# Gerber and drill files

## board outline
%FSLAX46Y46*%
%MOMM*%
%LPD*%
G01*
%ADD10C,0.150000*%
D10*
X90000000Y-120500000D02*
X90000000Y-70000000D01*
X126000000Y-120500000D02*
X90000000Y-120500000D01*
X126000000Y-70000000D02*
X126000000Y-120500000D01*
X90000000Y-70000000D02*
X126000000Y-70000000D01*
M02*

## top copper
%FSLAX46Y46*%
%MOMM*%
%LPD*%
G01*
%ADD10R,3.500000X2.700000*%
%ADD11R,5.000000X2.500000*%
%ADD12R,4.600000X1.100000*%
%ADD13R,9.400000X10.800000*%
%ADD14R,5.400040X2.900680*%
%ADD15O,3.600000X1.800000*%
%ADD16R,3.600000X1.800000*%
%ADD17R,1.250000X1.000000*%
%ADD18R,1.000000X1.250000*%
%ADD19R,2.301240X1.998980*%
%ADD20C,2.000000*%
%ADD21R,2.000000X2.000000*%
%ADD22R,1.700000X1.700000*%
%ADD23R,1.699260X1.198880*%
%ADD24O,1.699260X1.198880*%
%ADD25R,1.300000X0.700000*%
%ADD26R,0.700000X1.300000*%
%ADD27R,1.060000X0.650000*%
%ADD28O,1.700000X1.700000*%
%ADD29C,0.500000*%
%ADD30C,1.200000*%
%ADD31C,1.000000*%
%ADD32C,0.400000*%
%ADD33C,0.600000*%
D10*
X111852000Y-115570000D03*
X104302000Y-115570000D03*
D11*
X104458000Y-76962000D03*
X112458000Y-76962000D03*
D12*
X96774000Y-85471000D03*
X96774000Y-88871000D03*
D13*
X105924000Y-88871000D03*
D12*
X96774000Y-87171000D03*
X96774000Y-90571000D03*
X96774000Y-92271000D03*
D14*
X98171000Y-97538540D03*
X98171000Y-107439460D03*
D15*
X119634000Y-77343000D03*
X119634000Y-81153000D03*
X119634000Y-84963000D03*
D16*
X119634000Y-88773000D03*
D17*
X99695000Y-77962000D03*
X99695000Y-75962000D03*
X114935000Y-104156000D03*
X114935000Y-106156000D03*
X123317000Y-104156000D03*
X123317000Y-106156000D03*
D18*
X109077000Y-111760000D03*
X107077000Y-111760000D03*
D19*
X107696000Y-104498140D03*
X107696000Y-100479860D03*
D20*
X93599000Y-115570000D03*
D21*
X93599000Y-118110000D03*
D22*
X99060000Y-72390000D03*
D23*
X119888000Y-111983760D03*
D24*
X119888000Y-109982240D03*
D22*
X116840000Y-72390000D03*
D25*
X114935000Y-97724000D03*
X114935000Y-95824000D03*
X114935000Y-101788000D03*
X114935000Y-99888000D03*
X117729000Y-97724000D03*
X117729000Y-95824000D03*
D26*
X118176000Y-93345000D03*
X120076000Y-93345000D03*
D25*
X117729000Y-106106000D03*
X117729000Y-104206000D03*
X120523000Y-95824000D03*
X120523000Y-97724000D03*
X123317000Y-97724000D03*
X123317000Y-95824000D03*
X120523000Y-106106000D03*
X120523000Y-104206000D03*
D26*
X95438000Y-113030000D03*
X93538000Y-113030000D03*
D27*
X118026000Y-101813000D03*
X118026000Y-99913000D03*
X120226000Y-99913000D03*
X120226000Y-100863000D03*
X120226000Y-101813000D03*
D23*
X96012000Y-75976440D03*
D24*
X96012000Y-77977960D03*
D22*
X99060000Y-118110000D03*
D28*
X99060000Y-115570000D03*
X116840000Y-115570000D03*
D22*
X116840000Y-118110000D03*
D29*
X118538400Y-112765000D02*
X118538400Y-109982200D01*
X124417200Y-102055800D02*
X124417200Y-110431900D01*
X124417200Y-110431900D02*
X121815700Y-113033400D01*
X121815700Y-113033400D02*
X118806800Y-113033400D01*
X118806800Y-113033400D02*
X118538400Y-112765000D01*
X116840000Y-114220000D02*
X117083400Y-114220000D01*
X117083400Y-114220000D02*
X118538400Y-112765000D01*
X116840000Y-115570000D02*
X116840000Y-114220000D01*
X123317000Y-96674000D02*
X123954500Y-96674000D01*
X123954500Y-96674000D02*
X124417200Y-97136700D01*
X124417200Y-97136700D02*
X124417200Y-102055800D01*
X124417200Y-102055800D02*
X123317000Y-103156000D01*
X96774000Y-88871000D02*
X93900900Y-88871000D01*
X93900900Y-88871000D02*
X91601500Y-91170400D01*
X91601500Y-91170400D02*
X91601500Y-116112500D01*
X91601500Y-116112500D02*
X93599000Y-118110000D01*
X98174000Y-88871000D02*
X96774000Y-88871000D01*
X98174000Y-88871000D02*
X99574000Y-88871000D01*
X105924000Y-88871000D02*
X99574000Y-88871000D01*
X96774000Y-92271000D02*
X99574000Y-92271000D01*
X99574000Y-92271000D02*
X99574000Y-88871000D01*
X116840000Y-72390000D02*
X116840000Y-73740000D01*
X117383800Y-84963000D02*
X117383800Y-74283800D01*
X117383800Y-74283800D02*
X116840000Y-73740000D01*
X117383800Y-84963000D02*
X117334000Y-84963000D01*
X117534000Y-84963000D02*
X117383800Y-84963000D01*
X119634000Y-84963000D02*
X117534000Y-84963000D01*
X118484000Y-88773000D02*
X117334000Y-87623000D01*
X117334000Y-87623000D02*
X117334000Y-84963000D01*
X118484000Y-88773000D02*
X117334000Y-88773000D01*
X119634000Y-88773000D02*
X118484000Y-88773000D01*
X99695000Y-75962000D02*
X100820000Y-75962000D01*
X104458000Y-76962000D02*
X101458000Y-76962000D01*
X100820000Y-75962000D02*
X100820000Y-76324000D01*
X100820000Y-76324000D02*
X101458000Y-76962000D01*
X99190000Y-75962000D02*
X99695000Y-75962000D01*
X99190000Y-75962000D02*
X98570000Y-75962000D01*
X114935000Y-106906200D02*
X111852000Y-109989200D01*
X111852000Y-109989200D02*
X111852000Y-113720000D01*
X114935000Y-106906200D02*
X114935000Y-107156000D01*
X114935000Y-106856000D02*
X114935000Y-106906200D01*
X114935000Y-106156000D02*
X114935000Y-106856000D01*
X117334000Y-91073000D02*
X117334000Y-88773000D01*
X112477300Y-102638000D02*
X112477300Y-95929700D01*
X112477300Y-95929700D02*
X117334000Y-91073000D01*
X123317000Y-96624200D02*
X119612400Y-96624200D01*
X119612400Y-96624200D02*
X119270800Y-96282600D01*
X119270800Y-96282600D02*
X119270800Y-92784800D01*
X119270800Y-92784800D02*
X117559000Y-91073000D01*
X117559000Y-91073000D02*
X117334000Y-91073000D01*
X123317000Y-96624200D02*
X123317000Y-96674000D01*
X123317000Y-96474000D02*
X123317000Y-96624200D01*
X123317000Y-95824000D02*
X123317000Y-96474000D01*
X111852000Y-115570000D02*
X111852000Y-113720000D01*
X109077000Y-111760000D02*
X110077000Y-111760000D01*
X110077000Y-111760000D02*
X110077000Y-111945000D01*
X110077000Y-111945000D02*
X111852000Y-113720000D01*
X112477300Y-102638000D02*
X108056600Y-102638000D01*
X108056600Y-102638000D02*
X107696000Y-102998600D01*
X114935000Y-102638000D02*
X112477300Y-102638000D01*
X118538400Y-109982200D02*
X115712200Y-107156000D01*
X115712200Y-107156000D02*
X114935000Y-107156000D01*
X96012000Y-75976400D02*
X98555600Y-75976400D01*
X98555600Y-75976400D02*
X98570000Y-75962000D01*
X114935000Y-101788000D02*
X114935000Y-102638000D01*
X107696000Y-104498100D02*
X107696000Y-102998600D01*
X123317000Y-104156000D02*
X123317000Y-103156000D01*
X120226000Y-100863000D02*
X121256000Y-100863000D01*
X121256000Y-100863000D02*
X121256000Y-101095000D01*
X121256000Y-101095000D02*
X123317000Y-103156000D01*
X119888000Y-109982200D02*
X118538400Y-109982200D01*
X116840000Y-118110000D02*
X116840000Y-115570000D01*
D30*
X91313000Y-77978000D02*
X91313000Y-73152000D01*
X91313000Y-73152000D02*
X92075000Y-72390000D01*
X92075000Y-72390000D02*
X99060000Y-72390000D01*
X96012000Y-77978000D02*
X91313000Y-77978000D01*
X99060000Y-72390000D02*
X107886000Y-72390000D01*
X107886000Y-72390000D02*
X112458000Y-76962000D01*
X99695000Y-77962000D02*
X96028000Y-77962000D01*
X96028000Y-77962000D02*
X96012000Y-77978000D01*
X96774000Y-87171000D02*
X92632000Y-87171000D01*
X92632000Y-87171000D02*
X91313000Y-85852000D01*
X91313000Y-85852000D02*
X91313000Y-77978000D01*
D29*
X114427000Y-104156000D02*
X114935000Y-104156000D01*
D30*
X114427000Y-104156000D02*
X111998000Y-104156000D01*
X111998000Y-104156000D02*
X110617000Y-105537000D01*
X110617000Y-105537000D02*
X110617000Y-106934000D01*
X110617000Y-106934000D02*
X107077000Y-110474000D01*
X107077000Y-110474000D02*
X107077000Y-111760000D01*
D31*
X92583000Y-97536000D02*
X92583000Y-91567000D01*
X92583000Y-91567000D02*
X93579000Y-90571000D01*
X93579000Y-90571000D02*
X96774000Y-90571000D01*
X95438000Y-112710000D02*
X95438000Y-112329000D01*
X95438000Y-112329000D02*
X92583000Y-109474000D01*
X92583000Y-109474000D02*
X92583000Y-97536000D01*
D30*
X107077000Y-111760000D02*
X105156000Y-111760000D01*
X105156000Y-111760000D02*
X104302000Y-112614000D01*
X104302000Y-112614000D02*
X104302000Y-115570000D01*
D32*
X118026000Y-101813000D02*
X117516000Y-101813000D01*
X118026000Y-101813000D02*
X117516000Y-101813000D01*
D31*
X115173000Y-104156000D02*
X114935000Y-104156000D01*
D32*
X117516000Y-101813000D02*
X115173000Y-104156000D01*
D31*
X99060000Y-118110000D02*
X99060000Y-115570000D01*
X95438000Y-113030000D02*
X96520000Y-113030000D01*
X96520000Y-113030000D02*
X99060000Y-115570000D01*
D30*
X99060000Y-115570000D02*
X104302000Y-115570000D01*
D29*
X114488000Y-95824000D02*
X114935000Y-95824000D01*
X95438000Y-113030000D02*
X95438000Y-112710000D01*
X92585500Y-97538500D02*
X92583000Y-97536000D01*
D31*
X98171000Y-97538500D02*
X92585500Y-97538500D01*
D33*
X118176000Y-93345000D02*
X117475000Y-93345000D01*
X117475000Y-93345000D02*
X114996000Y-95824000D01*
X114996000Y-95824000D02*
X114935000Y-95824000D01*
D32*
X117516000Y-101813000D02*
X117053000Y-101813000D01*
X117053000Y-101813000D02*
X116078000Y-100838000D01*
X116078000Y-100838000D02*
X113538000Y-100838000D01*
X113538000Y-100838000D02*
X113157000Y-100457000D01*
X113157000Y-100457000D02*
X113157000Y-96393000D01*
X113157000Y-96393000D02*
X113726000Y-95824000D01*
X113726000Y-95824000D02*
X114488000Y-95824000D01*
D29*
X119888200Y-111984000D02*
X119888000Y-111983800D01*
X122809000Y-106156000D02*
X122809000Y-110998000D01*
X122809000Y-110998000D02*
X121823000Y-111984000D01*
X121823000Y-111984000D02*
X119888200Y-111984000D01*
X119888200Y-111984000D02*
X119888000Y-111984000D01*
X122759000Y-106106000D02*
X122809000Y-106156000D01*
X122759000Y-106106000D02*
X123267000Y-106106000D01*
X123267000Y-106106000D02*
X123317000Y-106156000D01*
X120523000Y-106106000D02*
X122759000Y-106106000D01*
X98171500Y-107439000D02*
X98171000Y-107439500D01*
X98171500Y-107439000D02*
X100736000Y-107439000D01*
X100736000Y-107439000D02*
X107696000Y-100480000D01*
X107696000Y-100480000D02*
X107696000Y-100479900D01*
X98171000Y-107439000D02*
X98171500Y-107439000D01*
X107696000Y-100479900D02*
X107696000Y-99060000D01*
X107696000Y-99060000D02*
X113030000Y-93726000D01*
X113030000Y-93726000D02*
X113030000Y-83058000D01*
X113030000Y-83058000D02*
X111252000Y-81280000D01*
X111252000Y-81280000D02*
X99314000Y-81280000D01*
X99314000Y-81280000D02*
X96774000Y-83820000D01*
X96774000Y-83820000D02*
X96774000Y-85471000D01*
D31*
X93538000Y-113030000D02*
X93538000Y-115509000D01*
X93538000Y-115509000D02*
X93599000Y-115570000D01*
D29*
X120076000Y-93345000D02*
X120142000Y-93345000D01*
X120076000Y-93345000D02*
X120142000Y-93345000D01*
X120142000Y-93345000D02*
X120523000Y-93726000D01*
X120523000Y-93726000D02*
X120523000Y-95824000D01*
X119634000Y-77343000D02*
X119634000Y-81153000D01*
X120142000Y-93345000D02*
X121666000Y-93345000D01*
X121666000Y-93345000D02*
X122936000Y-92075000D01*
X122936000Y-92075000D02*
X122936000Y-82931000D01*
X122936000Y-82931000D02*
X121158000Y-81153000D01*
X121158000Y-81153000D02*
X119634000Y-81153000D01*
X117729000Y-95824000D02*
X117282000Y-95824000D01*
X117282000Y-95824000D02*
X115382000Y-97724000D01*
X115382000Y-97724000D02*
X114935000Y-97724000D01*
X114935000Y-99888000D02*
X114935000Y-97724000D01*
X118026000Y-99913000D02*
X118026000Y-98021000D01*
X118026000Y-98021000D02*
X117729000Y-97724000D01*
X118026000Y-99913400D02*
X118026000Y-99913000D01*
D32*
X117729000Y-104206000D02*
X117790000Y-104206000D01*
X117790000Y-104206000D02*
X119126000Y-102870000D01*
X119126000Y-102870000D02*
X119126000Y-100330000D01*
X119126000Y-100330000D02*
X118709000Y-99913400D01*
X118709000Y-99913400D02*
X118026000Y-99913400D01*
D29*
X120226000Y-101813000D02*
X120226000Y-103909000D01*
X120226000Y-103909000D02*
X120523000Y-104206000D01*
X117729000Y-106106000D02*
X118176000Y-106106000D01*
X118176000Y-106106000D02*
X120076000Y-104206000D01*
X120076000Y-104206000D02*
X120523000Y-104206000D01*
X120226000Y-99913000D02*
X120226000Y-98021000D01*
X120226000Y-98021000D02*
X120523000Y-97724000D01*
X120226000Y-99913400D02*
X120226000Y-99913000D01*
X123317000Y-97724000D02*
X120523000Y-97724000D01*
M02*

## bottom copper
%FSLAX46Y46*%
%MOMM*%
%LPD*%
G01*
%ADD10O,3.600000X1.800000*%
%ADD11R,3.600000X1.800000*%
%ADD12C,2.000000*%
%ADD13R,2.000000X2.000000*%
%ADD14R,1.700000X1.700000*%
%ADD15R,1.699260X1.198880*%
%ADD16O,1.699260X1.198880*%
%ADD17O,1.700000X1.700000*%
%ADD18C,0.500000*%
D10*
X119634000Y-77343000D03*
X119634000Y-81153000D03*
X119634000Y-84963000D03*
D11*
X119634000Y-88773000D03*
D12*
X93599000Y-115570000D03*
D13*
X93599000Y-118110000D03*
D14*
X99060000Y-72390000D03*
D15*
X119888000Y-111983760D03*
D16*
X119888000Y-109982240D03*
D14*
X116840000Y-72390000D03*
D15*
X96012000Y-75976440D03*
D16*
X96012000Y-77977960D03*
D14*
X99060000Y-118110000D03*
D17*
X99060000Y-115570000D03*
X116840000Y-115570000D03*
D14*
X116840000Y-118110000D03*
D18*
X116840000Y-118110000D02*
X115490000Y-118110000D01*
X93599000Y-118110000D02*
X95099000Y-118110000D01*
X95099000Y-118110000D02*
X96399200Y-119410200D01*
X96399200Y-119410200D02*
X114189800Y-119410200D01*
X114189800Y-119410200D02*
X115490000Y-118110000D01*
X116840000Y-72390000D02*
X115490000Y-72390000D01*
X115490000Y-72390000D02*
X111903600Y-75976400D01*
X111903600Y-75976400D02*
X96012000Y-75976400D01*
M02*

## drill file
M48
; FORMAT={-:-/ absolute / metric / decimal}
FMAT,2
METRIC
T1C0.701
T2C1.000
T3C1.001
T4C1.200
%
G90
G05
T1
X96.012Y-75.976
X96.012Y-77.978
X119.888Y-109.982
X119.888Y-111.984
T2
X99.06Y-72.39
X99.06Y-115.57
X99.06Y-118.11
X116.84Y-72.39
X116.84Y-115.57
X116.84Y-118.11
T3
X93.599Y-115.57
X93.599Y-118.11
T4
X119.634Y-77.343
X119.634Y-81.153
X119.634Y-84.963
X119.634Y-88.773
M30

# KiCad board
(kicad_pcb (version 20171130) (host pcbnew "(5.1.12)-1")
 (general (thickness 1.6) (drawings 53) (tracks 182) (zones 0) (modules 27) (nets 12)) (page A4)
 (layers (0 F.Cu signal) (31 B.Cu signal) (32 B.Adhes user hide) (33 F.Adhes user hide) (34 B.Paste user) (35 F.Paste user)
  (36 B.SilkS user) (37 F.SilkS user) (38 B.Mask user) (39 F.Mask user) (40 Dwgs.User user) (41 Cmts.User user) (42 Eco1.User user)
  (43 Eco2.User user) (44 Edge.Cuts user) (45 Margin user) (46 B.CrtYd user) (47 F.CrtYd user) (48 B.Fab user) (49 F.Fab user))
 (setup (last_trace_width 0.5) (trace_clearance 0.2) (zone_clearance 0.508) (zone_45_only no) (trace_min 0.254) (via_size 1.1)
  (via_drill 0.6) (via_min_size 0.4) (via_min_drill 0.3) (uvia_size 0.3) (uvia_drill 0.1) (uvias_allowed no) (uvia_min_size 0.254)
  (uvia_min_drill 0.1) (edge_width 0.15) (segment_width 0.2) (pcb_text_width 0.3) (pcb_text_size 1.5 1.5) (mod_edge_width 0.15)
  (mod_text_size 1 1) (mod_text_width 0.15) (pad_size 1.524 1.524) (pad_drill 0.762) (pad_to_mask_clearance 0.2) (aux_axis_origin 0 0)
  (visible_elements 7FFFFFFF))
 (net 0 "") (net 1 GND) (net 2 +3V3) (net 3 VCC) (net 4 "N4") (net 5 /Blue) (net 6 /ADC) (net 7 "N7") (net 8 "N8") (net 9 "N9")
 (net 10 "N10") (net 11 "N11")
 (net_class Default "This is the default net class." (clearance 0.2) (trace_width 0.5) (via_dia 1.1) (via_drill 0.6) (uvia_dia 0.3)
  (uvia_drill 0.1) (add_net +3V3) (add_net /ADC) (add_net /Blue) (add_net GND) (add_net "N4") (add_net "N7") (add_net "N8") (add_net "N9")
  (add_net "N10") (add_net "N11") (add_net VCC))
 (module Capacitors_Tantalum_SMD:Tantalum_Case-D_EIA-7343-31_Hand (layer F.Cu) (at 108.077 115.57)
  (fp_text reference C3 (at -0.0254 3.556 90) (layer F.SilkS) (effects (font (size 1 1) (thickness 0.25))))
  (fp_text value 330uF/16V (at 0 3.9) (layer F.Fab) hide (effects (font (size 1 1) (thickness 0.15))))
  (pad 2 smd rect (at 3.775 0) (size 3.5 2.7) (layers F.Cu F.Paste F.Mask) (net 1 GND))
  (pad 1 smd rect (at -3.775 0) (size 3.5 2.7) (layers F.Cu F.Paste F.Mask) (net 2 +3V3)))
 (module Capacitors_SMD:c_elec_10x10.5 (layer F.Cu) (at 108.458 76.962 180)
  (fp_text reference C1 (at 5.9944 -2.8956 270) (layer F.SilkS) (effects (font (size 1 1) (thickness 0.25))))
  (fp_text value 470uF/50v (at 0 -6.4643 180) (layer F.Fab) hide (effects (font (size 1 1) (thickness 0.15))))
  (pad 2 smd rect (at 4 0) (size 5 2.5) (layers F.Cu F.Paste F.Mask) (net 1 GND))
  (pad 1 smd rect (at -4 0) (size 5 2.5) (layers F.Cu F.Paste F.Mask) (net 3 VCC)))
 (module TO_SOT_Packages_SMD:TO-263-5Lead (layer F.Cu) (at 96.774 88.871)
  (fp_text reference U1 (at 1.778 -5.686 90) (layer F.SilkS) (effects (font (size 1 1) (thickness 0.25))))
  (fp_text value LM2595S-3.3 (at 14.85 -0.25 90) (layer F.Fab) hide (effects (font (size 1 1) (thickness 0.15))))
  (pad 1 smd rect (at 0 -3.4) (size 4.6 1.1) (layers F.Cu F.Paste F.Mask) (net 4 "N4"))
  (pad 3 smd rect (at 0 0) (size 4.6 1.1) (layers F.Cu F.Paste F.Mask) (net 1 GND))
  (pad 3 smd rect (at 9.15 0) (size 9.4 10.8) (layers F.Cu F.Paste F.Mask) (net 1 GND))
  (pad 2 smd rect (at 0 -1.7) (size 4.6 1.1) (layers F.Cu F.Paste F.Mask) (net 3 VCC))
  (pad 4 smd rect (at 0 1.7) (size 4.6 1.1) (layers F.Cu F.Paste F.Mask) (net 2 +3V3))
  (pad 5 smd rect (at 0 3.4) (size 4.6 1.1) (layers F.Cu F.Paste F.Mask) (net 1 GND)))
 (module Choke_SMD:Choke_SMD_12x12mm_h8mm (layer F.Cu) (at 98.171 102.489 90)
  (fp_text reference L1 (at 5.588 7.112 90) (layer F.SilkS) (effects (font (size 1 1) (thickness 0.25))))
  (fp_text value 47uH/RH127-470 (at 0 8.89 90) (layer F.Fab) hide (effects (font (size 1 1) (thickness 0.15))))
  (pad 2 smd rect (at 4.95046 0 90) (size 2.90068 5.40004) (layers F.Cu F.Paste F.Mask) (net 2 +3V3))
  (pad 1 smd rect (at -4.95046 0 90) (size 2.90068 5.40004) (layers F.Cu F.Paste F.Mask) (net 4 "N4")))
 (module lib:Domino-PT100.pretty (layer F.Cu) (at 119.634 88.773 90)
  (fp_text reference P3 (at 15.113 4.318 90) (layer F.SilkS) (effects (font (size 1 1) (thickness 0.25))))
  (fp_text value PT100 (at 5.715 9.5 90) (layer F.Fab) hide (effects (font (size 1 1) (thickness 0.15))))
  (pad 4 thru_hole oval (at 11.43 0 90) (size 1.8 3.6) (drill 1.2) (layers *.Cu *.Mask) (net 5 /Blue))
  (pad 3 thru_hole oval (at 7.62 0 90) (size 1.8 3.6) (drill 1.2) (layers *.Cu *.Mask) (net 5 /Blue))
  (pad 2 thru_hole oval (at 3.81 0 90) (size 1.8 3.6) (drill 1.2) (layers *.Cu *.Mask) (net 1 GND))
  (pad 1 thru_hole rect (at 0 0 90) (size 1.8 3.6) (drill 1.2) (layers *.Cu *.Mask) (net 1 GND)))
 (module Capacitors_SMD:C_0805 (layer F.Cu) (at 99.695 76.962 90)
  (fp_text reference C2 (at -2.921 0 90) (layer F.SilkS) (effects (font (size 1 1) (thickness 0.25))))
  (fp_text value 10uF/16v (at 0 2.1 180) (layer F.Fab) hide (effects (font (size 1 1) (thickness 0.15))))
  (pad 1 smd rect (at -1 0 90) (size 1 1.25) (layers F.Cu F.Paste F.Mask) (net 3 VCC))
  (pad 2 smd rect (at 1 0 90) (size 1 1.25) (layers F.Cu F.Paste F.Mask) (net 1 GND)))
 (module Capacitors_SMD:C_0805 (layer F.Cu) (at 114.935 105.156 270)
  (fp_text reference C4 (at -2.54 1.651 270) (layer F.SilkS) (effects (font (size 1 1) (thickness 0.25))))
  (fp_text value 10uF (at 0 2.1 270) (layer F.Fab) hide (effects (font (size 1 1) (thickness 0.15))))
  (pad 1 smd rect (at -1 0 270) (size 1 1.25) (layers F.Cu F.Paste F.Mask) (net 2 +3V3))
  (pad 2 smd rect (at 1 0 270) (size 1 1.25) (layers F.Cu F.Paste F.Mask) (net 1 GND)))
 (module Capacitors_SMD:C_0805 (layer F.Cu) (at 123.317 105.156 90)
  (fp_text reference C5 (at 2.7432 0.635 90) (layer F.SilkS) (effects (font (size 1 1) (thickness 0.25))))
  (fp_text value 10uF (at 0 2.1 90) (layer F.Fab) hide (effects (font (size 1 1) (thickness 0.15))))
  (pad 2 smd rect (at 1 0 90) (size 1 1.25) (layers F.Cu F.Paste F.Mask) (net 1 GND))
  (pad 1 smd rect (at -1 0 90) (size 1 1.25) (layers F.Cu F.Paste F.Mask) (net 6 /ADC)))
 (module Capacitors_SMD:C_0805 (layer F.Cu) (at 108.077 111.76)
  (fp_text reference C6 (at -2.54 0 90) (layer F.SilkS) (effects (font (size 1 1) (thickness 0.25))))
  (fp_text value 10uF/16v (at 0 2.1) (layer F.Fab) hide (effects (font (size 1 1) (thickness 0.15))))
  (pad 2 smd rect (at 1 0) (size 1 1.25) (layers F.Cu F.Paste F.Mask) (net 1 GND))
  (pad 1 smd rect (at -1 0) (size 1 1.25) (layers F.Cu F.Paste F.Mask) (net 2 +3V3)))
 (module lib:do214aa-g (layer F.Cu) (at 107.696 102.489 270)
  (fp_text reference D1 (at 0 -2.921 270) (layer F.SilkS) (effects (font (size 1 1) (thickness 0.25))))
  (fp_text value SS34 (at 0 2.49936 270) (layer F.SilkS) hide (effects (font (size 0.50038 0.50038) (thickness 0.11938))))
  (pad 2 smd rect (at 2.00914 0 270) (size 1.99898 2.30124) (layers F.Cu F.Paste F.Mask) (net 1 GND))
  (pad 1 smd rect (at -2.00914 0 270) (size 1.99898 2.30124) (layers F.Cu F.Paste F.Mask) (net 4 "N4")))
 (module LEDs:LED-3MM (layer F.Cu) (at 93.599 118.11 90)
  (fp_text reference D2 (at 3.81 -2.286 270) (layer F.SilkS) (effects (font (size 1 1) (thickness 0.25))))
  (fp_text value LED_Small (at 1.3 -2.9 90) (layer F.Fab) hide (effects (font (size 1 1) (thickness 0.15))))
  (pad 2 thru_hole circle (at 2.54 0 90) (size 2 2) (drill 1.00076) (layers *.Cu *.Mask) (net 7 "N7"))
  (pad 1 thru_hole rect (at 0 0 180) (size 2 2) (drill 1.00076) (layers *.Cu *.Mask) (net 1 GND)))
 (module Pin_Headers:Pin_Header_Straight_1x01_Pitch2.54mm (layer F.Cu) (at 99.06 72.39)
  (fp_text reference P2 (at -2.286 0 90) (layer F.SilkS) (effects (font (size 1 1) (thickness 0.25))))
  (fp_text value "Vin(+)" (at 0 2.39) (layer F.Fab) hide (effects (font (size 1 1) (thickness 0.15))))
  (pad 1 thru_hole rect (at 0 0) (size 1.7 1.7) (drill 1) (layers *.Cu *.Mask) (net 3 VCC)))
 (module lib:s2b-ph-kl (layer F.Cu) (at 119.888 110.983 90)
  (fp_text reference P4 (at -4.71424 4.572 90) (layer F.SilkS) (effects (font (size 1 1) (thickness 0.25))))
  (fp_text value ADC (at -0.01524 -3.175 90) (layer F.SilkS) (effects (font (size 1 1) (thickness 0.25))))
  (pad 1 thru_hole rect (at -1.00076 0 90) (size 1.19888 1.69926) (drill 0.70104) (layers *.Cu *.Mask F.SilkS) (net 6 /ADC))
  (pad 2 thru_hole oval (at 1.00076 0 90) (size 1.19888 1.69926) (drill 0.70104) (layers *.Cu *.Mask F.SilkS) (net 1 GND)))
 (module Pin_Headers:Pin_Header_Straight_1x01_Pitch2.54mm (layer F.Cu) (at 116.84 72.39)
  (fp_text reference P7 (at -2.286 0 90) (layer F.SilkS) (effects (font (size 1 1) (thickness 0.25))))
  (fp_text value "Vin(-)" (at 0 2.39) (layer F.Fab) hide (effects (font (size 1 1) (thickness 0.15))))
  (pad 1 thru_hole rect (at 0 0) (size 1.7 1.7) (drill 1) (layers *.Cu *.Mask) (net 1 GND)))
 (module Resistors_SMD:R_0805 (layer F.Cu) (at 114.935 96.774 270)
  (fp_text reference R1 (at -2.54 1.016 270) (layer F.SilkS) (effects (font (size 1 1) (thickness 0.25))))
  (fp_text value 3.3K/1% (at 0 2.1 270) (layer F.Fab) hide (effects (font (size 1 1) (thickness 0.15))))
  (pad 2 smd rect (at 0.95 0 270) (size 0.7 1.3) (layers F.Cu F.Paste F.Mask) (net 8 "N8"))
  (pad 1 smd rect (at -0.95 0 270) (size 0.7 1.3) (layers F.Cu F.Paste F.Mask) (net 2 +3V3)))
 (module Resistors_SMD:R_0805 (layer F.Cu) (at 114.935 100.838 270)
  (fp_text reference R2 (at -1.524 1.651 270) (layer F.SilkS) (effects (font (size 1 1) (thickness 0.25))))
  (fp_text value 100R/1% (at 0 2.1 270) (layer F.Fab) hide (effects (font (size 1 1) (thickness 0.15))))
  (pad 2 smd rect (at 0.95 0 270) (size 0.7 1.3) (layers F.Cu F.Paste F.Mask) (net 1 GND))
  (pad 1 smd rect (at -0.95 0 270) (size 0.7 1.3) (layers F.Cu F.Paste F.Mask) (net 8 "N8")))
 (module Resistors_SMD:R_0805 (layer F.Cu) (at 117.729 96.774 90)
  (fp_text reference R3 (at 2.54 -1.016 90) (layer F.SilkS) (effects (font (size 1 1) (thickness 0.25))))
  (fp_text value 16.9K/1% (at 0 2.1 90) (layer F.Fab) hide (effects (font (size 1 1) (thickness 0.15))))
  (pad 1 smd rect (at -0.95 0 90) (size 0.7 1.3) (layers F.Cu F.Paste F.Mask) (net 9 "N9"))
  (pad 2 smd rect (at 0.95 0 90) (size 0.7 1.3) (layers F.Cu F.Paste F.Mask) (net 8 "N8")))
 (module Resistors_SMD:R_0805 (layer F.Cu) (at 119.126 93.345)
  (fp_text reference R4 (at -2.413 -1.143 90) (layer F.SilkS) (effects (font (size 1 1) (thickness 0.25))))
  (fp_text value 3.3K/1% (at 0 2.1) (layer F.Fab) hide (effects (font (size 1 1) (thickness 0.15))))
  (pad 1 smd rect (at -0.95 0) (size 0.7 1.3) (layers F.Cu F.Paste F.Mask) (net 2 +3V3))
  (pad 2 smd rect (at 0.95 0) (size 0.7 1.3) (layers F.Cu F.Paste F.Mask) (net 5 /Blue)))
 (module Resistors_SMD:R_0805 (layer F.Cu) (at 117.729 105.156 270)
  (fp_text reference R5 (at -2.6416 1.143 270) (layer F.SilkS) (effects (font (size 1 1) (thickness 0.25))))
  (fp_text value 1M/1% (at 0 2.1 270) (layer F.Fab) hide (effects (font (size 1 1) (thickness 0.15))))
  (pad 2 smd rect (at 0.95 0 270) (size 0.7 1.3) (layers F.Cu F.Paste F.Mask) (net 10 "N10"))
  (pad 1 smd rect (at -0.95 0 270) (size 0.7 1.3) (layers F.Cu F.Paste F.Mask) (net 9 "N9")))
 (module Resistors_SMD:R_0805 (layer F.Cu) (at 120.523 96.774 90)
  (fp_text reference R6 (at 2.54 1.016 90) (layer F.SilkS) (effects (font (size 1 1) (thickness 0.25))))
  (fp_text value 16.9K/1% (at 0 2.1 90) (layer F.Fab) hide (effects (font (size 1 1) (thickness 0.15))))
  (pad 2 smd rect (at 0.95 0 90) (size 0.7 1.3) (layers F.Cu F.Paste F.Mask) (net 5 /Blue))
  (pad 1 smd rect (at -0.95 0 90) (size 0.7 1.3) (layers F.Cu F.Paste F.Mask) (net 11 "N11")))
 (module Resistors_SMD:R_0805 (layer F.Cu) (at 123.317 96.774 270)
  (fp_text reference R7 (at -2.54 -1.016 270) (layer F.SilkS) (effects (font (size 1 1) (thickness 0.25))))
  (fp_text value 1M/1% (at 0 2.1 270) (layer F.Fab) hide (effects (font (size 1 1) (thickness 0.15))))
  (pad 2 smd rect (at 0.95 0 270) (size 0.7 1.3) (layers F.Cu F.Paste F.Mask) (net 11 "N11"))
  (pad 1 smd rect (at -0.95 0 270) (size 0.7 1.3) (layers F.Cu F.Paste F.Mask) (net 1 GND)))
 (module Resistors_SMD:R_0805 (layer F.Cu) (at 120.523 105.156 90)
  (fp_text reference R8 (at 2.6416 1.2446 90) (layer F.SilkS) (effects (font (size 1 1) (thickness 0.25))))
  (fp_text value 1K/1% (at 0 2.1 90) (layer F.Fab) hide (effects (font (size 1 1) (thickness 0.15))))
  (pad 1 smd rect (at -0.95 0 90) (size 0.7 1.3) (layers F.Cu F.Paste F.Mask) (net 6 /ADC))
  (pad 2 smd rect (at 0.95 0 90) (size 0.7 1.3) (layers F.Cu F.Paste F.Mask) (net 10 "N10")))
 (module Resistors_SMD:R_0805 (layer F.Cu) (at 94.488 113.03 180)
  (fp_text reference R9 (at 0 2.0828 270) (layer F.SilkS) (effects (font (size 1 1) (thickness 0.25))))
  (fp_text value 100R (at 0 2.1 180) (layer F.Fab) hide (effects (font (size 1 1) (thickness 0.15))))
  (pad 1 smd rect (at -0.95 0 180) (size 0.7 1.3) (layers F.Cu F.Paste F.Mask) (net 2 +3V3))
  (pad 2 smd rect (at 0.95 0 180) (size 0.7 1.3) (layers F.Cu F.Paste F.Mask) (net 7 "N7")))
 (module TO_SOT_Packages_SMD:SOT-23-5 (layer F.Cu) (at 119.126 100.863 180)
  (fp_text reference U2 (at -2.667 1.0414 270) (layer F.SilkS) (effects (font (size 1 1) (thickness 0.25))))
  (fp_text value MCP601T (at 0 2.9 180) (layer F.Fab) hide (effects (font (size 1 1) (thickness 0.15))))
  (pad 5 smd rect (at 1.1 -0.95 180) (size 1.06 0.65) (layers F.Cu F.Paste F.Mask) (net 2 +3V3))
  (pad 4 smd rect (at 1.1 0.95 180) (size 1.06 0.65) (layers F.Cu F.Paste F.Mask) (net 9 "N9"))
  (pad 3 smd rect (at -1.1 0.95 180) (size 1.06 0.65) (layers F.Cu F.Paste F.Mask) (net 11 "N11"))
  (pad 2 smd rect (at -1.1 0 180) (size 1.06 0.65) (layers F.Cu F.Paste F.Mask) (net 1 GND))
  (pad 1 smd rect (at -1.1 -0.95 180) (size 1.06 0.65) (layers F.Cu F.Paste F.Mask) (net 10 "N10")))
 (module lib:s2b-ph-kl (layer F.Cu) (at 96.012 76.9772 270)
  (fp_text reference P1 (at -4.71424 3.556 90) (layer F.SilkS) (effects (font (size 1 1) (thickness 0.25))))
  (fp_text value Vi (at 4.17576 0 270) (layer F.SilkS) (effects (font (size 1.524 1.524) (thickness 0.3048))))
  (pad 1 thru_hole rect (at -1.00076 0 270) (size 1.19888 1.69926) (drill 0.70104) (layers *.Cu *.Mask F.SilkS) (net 1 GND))
  (pad 2 thru_hole oval (at 1.00076 0 270) (size 1.19888 1.69926) (drill 0.70104) (layers *.Cu *.Mask F.SilkS) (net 3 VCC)))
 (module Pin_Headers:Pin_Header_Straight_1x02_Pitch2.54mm (layer F.Cu) (at 99.06 118.11 180)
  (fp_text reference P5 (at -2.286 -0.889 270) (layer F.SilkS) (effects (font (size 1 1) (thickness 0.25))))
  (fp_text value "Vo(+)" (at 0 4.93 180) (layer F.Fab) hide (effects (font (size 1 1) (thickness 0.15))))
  (pad 1 thru_hole rect (at 0 0 180) (size 1.7 1.7) (drill 1) (layers *.Cu *.Mask) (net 2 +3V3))
  (pad 2 thru_hole oval (at 0 2.54 180) (size 1.7 1.7) (drill 1) (layers *.Cu *.Mask) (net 2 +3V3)))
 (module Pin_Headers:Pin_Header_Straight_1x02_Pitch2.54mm (layer F.Cu) (at 116.84 118.11 180)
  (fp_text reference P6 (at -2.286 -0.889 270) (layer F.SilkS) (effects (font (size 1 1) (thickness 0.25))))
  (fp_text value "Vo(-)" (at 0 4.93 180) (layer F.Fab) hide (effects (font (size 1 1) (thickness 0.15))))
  (pad 2 thru_hole oval (at 0 2.54 180) (size 1.7 1.7) (drill 1) (layers *.Cu *.Mask) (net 1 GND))
  (pad 1 thru_hole rect (at 0 0 180) (size 1.7 1.7) (drill 1) (layers *.Cu *.Mask) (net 1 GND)))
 (gr_line (start 90 120.5) (end 90 70) (layer Edge.Cuts) (width 0.15))
 (gr_line (start 126 120.5) (end 90 120.5) (layer Edge.Cuts) (width 0.15))
 (gr_line (start 126 70) (end 126 120.5) (layer Edge.Cuts) (width 0.15))
 (gr_line (start 90 70) (end 126 70) (layer Edge.Cuts) (width 0.15))
 (segment (start 118.5384 112.765) (end 118.5384 109.9822) (width 0.5) (layer F.Cu) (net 1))
 (segment (start 124.4172 102.0558) (end 124.4172 110.4319) (width 0.5) (layer F.Cu) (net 1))
 (segment (start 124.4172 110.4319) (end 121.8157 113.0334) (width 0.5) (layer F.Cu) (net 1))
 (segment (start 121.8157 113.0334) (end 118.8068 113.0334) (width 0.5) (layer F.Cu) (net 1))
 (segment (start 118.8068 113.0334) (end 118.5384 112.765) (width 0.5) (layer F.Cu) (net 1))
 (segment (start 116.84 114.22) (end 117.0834 114.22) (width 0.5) (layer F.Cu) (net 1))
 (segment (start 117.0834 114.22) (end 118.5384 112.765) (width 0.5) (layer F.Cu) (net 1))
 (segment (start 116.84 115.57) (end 116.84 114.22) (width 0.5) (layer F.Cu) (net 1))
 (segment (start 123.317 96.674) (end 123.9545 96.674) (width 0.5) (layer F.Cu) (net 1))
 (segment (start 123.9545 96.674) (end 124.4172 97.1367) (width 0.5) (layer F.Cu) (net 1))
 (segment (start 124.4172 97.1367) (end 124.4172 102.0558) (width 0.5) (layer F.Cu) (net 1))
 (segment (start 124.4172 102.0558) (end 123.317 103.156) (width 0.5) (layer F.Cu) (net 1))
 (segment (start 96.774 88.871) (end 93.9009 88.871) (width 0.5) (layer F.Cu) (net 1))
 (segment (start 93.9009 88.871) (end 91.6015 91.1704) (width 0.5) (layer F.Cu) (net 1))
 (segment (start 91.6015 91.1704) (end 91.6015 116.1125) (width 0.5) (layer F.Cu) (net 1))
 (segment (start 91.6015 116.1125) (end 93.599 118.11) (width 0.5) (layer F.Cu) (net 1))
 (segment (start 98.174 88.871) (end 96.774 88.871) (width 0.5) (layer F.Cu) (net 1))
 (segment (start 98.174 88.871) (end 99.574 88.871) (width 0.5) (layer F.Cu) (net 1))
 (segment (start 105.924 88.871) (end 99.574 88.871) (width 0.5) (layer F.Cu) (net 1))
 (segment (start 96.774 92.271) (end 99.574 92.271) (width 0.5) (layer F.Cu) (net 1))
 (segment (start 99.574 92.271) (end 99.574 88.871) (width 0.5) (layer F.Cu) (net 1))
 (segment (start 116.84 72.39) (end 116.84 73.74) (width 0.5) (layer F.Cu) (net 1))
 (segment (start 117.3838 84.963) (end 117.3838 74.2838) (width 0.5) (layer F.Cu) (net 1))
 (segment (start 117.3838 74.2838) (end 116.84 73.74) (width 0.5) (layer F.Cu) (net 1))
 (segment (start 117.3838 84.963) (end 117.334 84.963) (width 0.5) (layer F.Cu) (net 1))
 (segment (start 117.534 84.963) (end 117.3838 84.963) (width 0.5) (layer F.Cu) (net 1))
 (segment (start 119.634 84.963) (end 117.534 84.963) (width 0.5) (layer F.Cu) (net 1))
 (segment (start 118.484 88.773) (end 117.334 87.623) (width 0.5) (layer F.Cu) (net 1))
 (segment (start 117.334 87.623) (end 117.334 84.963) (width 0.5) (layer F.Cu) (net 1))
 (segment (start 118.484 88.773) (end 117.334 88.773) (width 0.5) (layer F.Cu) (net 1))
 (segment (start 119.634 88.773) (end 118.484 88.773) (width 0.5) (layer F.Cu) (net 1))
 (segment (start 99.695 75.962) (end 100.82 75.962) (width 0.5) (layer F.Cu) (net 1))
 (segment (start 104.458 76.962) (end 101.458 76.962) (width 0.5) (layer F.Cu) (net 1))
 (segment (start 100.82 75.962) (end 100.82 76.324) (width 0.5) (layer F.Cu) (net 1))
 (segment (start 100.82 76.324) (end 101.458 76.962) (width 0.5) (layer F.Cu) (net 1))
 (segment (start 99.19 75.962) (end 99.695 75.962) (width 0.5) (layer F.Cu) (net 1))
 (segment (start 99.19 75.962) (end 98.57 75.962) (width 0.5) (layer F.Cu) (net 1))
 (segment (start 114.935 106.9062) (end 111.852 109.9892) (width 0.5) (layer F.Cu) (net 1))
 (segment (start 111.852 109.9892) (end 111.852 113.72) (width 0.5) (layer F.Cu) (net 1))
 (segment (start 114.935 106.9062) (end 114.935 107.156) (width 0.5) (layer F.Cu) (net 1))
 (segment (start 114.935 106.856) (end 114.935 106.9062) (width 0.5) (layer F.Cu) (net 1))
 (segment (start 114.935 106.156) (end 114.935 106.856) (width 0.5) (layer F.Cu) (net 1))
 (segment (start 117.334 91.073) (end 117.334 88.773) (width 0.5) (layer F.Cu) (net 1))
 (segment (start 112.4773 102.638) (end 112.4773 95.9297) (width 0.5) (layer F.Cu) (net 1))
 (segment (start 112.4773 95.9297) (end 117.334 91.073) (width 0.5) (layer F.Cu) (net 1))
 (segment (start 123.317 96.6242) (end 119.6124 96.6242) (width 0.5) (layer F.Cu) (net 1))
 (segment (start 119.6124 96.6242) (end 119.2708 96.2826) (width 0.5) (layer F.Cu) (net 1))
 (segment (start 119.2708 96.2826) (end 119.2708 92.7848) (width 0.5) (layer F.Cu) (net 1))
 (segment (start 119.2708 92.7848) (end 117.559 91.073) (width 0.5) (layer F.Cu) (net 1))
 (segment (start 117.559 91.073) (end 117.334 91.073) (width 0.5) (layer F.Cu) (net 1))
 (segment (start 123.317 96.6242) (end 123.317 96.674) (width 0.5) (layer F.Cu) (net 1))
 (segment (start 123.317 96.474) (end 123.317 96.6242) (width 0.5) (layer F.Cu) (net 1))
 (segment (start 123.317 95.824) (end 123.317 96.474) (width 0.5) (layer F.Cu) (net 1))
 (segment (start 111.852 115.57) (end 111.852 113.72) (width 0.5) (layer F.Cu) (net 1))
 (segment (start 109.077 111.76) (end 110.077 111.76) (width 0.5) (layer F.Cu) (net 1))
 (segment (start 110.077 111.76) (end 110.077 111.945) (width 0.5) (layer F.Cu) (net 1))
 (segment (start 110.077 111.945) (end 111.852 113.72) (width 0.5) (layer F.Cu) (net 1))
 (segment (start 112.4773 102.638) (end 108.0566 102.638) (width 0.5) (layer F.Cu) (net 1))
 (segment (start 108.0566 102.638) (end 107.696 102.9986) (width 0.5) (layer F.Cu) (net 1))
 (segment (start 114.935 102.638) (end 112.4773 102.638) (width 0.5) (layer F.Cu) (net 1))
 (segment (start 116.84 118.11) (end 115.49 118.11) (width 0.5) (layer B.Cu) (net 1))
 (segment (start 93.599 118.11) (end 95.099 118.11) (width 0.5) (layer B.Cu) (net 1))
 (segment (start 95.099 118.11) (end 96.3992 119.4102) (width 0.5) (layer B.Cu) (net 1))
 (segment (start 96.3992 119.4102) (end 114.1898 119.4102) (width 0.5) (layer B.Cu) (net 1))
 (segment (start 114.1898 119.4102) (end 115.49 118.11) (width 0.5) (layer B.Cu) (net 1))
 (segment (start 118.5384 109.9822) (end 115.7122 107.156) (width 0.5) (layer F.Cu) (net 1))
 (segment (start 115.7122 107.156) (end 114.935 107.156) (width 0.5) (layer F.Cu) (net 1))
 (segment (start 96.012 75.9764) (end 98.5556 75.9764) (width 0.5) (layer F.Cu) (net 1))
 (segment (start 98.5556 75.9764) (end 98.57 75.962) (width 0.5) (layer F.Cu) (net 1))
 (segment (start 116.84 72.39) (end 115.49 72.39) (width 0.5) (layer B.Cu) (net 1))
 (segment (start 115.49 72.39) (end 111.9036 75.9764) (width 0.5) (layer B.Cu) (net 1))
 (segment (start 111.9036 75.9764) (end 96.012 75.9764) (width 0.5) (layer B.Cu) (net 1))
 (segment (start 114.935 101.788) (end 114.935 102.638) (width 0.5) (layer F.Cu) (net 1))
 (segment (start 107.696 104.4981) (end 107.696 102.9986) (width 0.5) (layer F.Cu) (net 1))
 (segment (start 123.317 104.156) (end 123.317 103.156) (width 0.5) (layer F.Cu) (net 1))
 (segment (start 120.226 100.863) (end 121.256 100.863) (width 0.5) (layer F.Cu) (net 1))
 (segment (start 121.256 100.863) (end 121.256 101.095) (width 0.5) (layer F.Cu) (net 1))
 (segment (start 121.256 101.095) (end 123.317 103.156) (width 0.5) (layer F.Cu) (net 1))
 (segment (start 119.888 109.9822) (end 118.5384 109.9822) (width 0.5) (layer F.Cu) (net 1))
 (segment (start 116.84 118.11) (end 116.84 115.57) (width 0.5) (layer F.Cu) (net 1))
 (segment (start 91.313 77.978) (end 91.313 73.152) (width 1.2) (layer F.Cu) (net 3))
 (segment (start 91.313 73.152) (end 92.075 72.39) (width 1.2) (layer F.Cu) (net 3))
 (segment (start 92.075 72.39) (end 99.06 72.39) (width 1.2) (layer F.Cu) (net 3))
 (segment (start 96.012 77.978) (end 91.313 77.978) (width 1.2) (layer F.Cu) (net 3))
 (segment (start 99.06 72.39) (end 107.886 72.39) (width 1.2) (layer F.Cu) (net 3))
 (segment (start 107.886 72.39) (end 112.458 76.962) (width 1.2) (layer F.Cu) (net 3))
 (segment (start 99.695 77.962) (end 96.028 77.962) (width 1.2) (layer F.Cu) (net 3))
 (segment (start 96.028 77.962) (end 96.012 77.978) (width 1.2) (layer F.Cu) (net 3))
 (segment (start 96.774 87.171) (end 92.632 87.171) (width 1.2) (layer F.Cu) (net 3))
 (segment (start 92.632 87.171) (end 91.313 85.852) (width 1.2) (layer F.Cu) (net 3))
 (segment (start 91.313 85.852) (end 91.313 77.978) (width 1.2) (layer F.Cu) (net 3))
 (segment (start 114.427 104.156) (end 114.935 104.156) (width 0.5) (layer F.Cu) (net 2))
 (segment (start 114.427 104.156) (end 111.998 104.156) (width 1.2) (layer F.Cu) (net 2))
 (segment (start 111.998 104.156) (end 110.617 105.537) (width 1.2) (layer F.Cu) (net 2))
 (segment (start 110.617 105.537) (end 110.617 106.934) (width 1.2) (layer F.Cu) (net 2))
 (segment (start 110.617 106.934) (end 107.077 110.474) (width 1.2) (layer F.Cu) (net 2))
 (segment (start 107.077 110.474) (end 107.077 111.76) (width 1.2) (layer F.Cu) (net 2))
 (segment (start 92.583 97.536) (end 92.583 91.567) (width 1) (layer F.Cu) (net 2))
 (segment (start 92.583 91.567) (end 93.579 90.571) (width 1) (layer F.Cu) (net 2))
 (segment (start 93.579 90.571) (end 96.774 90.571) (width 1) (layer F.Cu) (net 2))
 (segment (start 95.438 112.71) (end 95.438 112.329) (width 1) (layer F.Cu) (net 2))
 (segment (start 95.438 112.329) (end 92.583 109.474) (width 1) (layer F.Cu) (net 2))
 (segment (start 92.583 109.474) (end 92.583 97.536) (width 1) (layer F.Cu) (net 2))
 (segment (start 107.077 111.76) (end 105.156 111.76) (width 1.2) (layer F.Cu) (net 2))
 (segment (start 105.156 111.76) (end 104.302 112.614) (width 1.2) (layer F.Cu) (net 2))
 (segment (start 104.302 112.614) (end 104.302 115.57) (width 1.2) (layer F.Cu) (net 2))
 (segment (start 118.026 101.813) (end 117.516 101.813) (width 0.4) (layer F.Cu) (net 2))
 (segment (start 118.026 101.813) (end 117.516 101.813) (width 0.4) (layer F.Cu) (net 2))
 (segment (start 115.173 104.156) (end 114.935 104.156) (width 1) (layer F.Cu) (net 2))
 (segment (start 117.516 101.813) (end 115.173 104.156) (width 0.4) (layer F.Cu) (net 2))
 (segment (start 99.06 118.11) (end 99.06 115.57) (width 1) (layer F.Cu) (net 2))
 (segment (start 95.438 113.03) (end 96.52 113.03) (width 1) (layer F.Cu) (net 2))
 (segment (start 96.52 113.03) (end 99.06 115.57) (width 1) (layer F.Cu) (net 2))
 (segment (start 99.06 115.57) (end 104.302 115.57) (width 1.2) (layer F.Cu) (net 2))
 (segment (start 114.488 95.824) (end 114.935 95.824) (width 0.5) (layer F.Cu) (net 2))
 (segment (start 95.438 113.03) (end 95.438 112.71) (width 0.5) (layer F.Cu) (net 2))
 (segment (start 92.5855 97.5385) (end 92.583 97.536) (width 0.5) (layer F.Cu) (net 2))
 (segment (start 98.171 97.5385) (end 92.5855 97.5385) (width 1) (layer F.Cu) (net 2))
 (segment (start 118.176 93.345) (end 117.475 93.345) (width 0.6) (layer F.Cu) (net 2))
 (segment (start 117.475 93.345) (end 114.996 95.824) (width 0.6) (layer F.Cu) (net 2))
 (segment (start 114.996 95.824) (end 114.935 95.824) (width 0.6) (layer F.Cu) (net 2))
 (segment (start 117.516 101.813) (end 117.053 101.813) (width 0.4) (layer F.Cu) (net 2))
 (segment (start 117.053 101.813) (end 116.078 100.838) (width 0.4) (layer F.Cu) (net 2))
 (segment (start 116.078 100.838) (end 113.538 100.838) (width 0.4) (layer F.Cu) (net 2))
 (segment (start 113.538 100.838) (end 113.157 100.457) (width 0.4) (layer F.Cu) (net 2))
 (segment (start 113.157 100.457) (end 113.157 96.393) (width 0.4) (layer F.Cu) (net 2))
 (segment (start 113.157 96.393) (end 113.726 95.824) (width 0.4) (layer F.Cu) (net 2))
 (segment (start 113.726 95.824) (end 114.488 95.824) (width 0.4) (layer F.Cu) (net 2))
 (segment (start 119.8882 111.984) (end 119.888 111.9838) (width 0.5) (layer F.Cu) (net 6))
 (segment (start 122.809 106.156) (end 122.809 110.998) (width 0.5) (layer F.Cu) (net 6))
 (segment (start 122.809 110.998) (end 121.823 111.984) (width 0.5) (layer F.Cu) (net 6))
 (segment (start 121.823 111.984) (end 119.8882 111.984) (width 0.5) (layer F.Cu) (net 6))
 (segment (start 119.8882 111.984) (end 119.888 111.984) (width 0.5) (layer F.Cu) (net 6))
 (segment (start 122.759 106.106) (end 122.809 106.156) (width 0.5) (layer F.Cu) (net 6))
 (segment (start 122.759 106.106) (end 123.267 106.106) (width 0.5) (layer F.Cu) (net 6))
 (segment (start 123.267 106.106) (end 123.317 106.156) (width 0.5) (layer F.Cu) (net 6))
 (segment (start 120.523 106.106) (end 122.759 106.106) (width 0.5) (layer F.Cu) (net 6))
 (segment (start 98.1715 107.439) (end 98.171 107.4395) (width 0.5) (layer F.Cu) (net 4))
 (segment (start 98.1715 107.439) (end 100.736 107.439) (width 0.5) (layer F.Cu) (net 4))
 (segment (start 100.736 107.439) (end 107.696 100.48) (width 0.5) (layer F.Cu) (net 4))
 (segment (start 107.696 100.48) (end 107.696 100.4799) (width 0.5) (layer F.Cu) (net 4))
 (segment (start 98.171 107.439) (end 98.1715 107.439) (width 0.5) (layer F.Cu) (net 4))
 (segment (start 107.696 100.4799) (end 107.696 99.06) (width 0.5) (layer F.Cu) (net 4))
 (segment (start 107.696 99.06) (end 113.03 93.726) (width 0.5) (layer F.Cu) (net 4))
 (segment (start 113.03 93.726) (end 113.03 83.058) (width 0.5) (layer F.Cu) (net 4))
 (segment (start 113.03 83.058) (end 111.252 81.28) (width 0.5) (layer F.Cu) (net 4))
 (segment (start 111.252 81.28) (end 99.314 81.28) (width 0.5) (layer F.Cu) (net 4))
 (segment (start 99.314 81.28) (end 96.774 83.82) (width 0.5) (layer F.Cu) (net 4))
 (segment (start 96.774 83.82) (end 96.774 85.471) (width 0.5) (layer F.Cu) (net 4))
 (segment (start 93.538 113.03) (end 93.538 115.509) (width 1) (layer F.Cu) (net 7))
 (segment (start 93.538 115.509) (end 93.599 115.57) (width 1) (layer F.Cu) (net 7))
 (segment (start 120.076 93.345) (end 120.142 93.345) (width 0.5) (layer F.Cu) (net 5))
 (segment (start 120.076 93.345) (end 120.142 93.345) (width 0.5) (layer F.Cu) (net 5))
 (segment (start 120.142 93.345) (end 120.523 93.726) (width 0.5) (layer F.Cu) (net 5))
 (segment (start 120.523 93.726) (end 120.523 95.824) (width 0.5) (layer F.Cu) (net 5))
 (segment (start 119.634 77.343) (end 119.634 81.153) (width 0.5) (layer F.Cu) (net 5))
 (segment (start 120.142 93.345) (end 121.666 93.345) (width 0.5) (layer F.Cu) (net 5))
 (segment (start 121.666 93.345) (end 122.936 92.075) (width 0.5) (layer F.Cu) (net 5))
 (segment (start 122.936 92.075) (end 122.936 82.931) (width 0.5) (layer F.Cu) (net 5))
 (segment (start 122.936 82.931) (end 121.158 81.153) (width 0.5) (layer F.Cu) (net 5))
 (segment (start 121.158 81.153) (end 119.634 81.153) (width 0.5) (layer F.Cu) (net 5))
 (segment (start 117.729 95.824) (end 117.282 95.824) (width 0.5) (layer F.Cu) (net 8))
 (segment (start 117.282 95.824) (end 115.382 97.724) (width 0.5) (layer F.Cu) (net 8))
 (segment (start 115.382 97.724) (end 114.935 97.724) (width 0.5) (layer F.Cu) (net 8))
 (segment (start 114.935 99.888) (end 114.935 97.724) (width 0.5) (layer F.Cu) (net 8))
 (segment (start 118.026 99.913) (end 118.026 98.021) (width 0.5) (layer F.Cu) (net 9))
 (segment (start 118.026 98.021) (end 117.729 97.724) (width 0.5) (layer F.Cu) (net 9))
 (segment (start 118.026 99.9134) (end 118.026 99.913) (width 0.5) (layer F.Cu) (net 9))
 (segment (start 117.729 104.206) (end 117.79 104.206) (width 0.4) (layer F.Cu) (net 9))
 (segment (start 117.79 104.206) (end 119.126 102.87) (width 0.4) (layer F.Cu) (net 9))
 (segment (start 119.126 102.87) (end 119.126 100.33) (width 0.4) (layer F.Cu) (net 9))
 (segment (start 119.126 100.33) (end 118.709 99.9134) (width 0.4) (layer F.Cu) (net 9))
 (segment (start 118.709 99.9134) (end 118.026 99.9134) (width 0.4) (layer F.Cu) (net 9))
 (segment (start 120.226 101.813) (end 120.226 103.909) (width 0.5) (layer F.Cu) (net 10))
 (segment (start 120.226 103.909) (end 120.523 104.206) (width 0.5) (layer F.Cu) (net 10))
 (segment (start 117.729 106.106) (end 118.176 106.106) (width 0.5) (layer F.Cu) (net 10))
 (segment (start 118.176 106.106) (end 120.076 104.206) (width 0.5) (layer F.Cu) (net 10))
 (segment (start 120.076 104.206) (end 120.523 104.206) (width 0.5) (layer F.Cu) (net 10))
 (segment (start 120.226 99.913) (end 120.226 98.021) (width 0.5) (layer F.Cu) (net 11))
 (segment (start 120.226 98.021) (end 120.523 97.724) (width 0.5) (layer F.Cu) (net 11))
 (segment (start 120.226 99.9134) (end 120.226 99.913) (width 0.5) (layer F.Cu) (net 11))
 (segment (start 123.317 97.724) (end 120.523 97.724) (width 0.5) (layer F.Cu) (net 11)))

